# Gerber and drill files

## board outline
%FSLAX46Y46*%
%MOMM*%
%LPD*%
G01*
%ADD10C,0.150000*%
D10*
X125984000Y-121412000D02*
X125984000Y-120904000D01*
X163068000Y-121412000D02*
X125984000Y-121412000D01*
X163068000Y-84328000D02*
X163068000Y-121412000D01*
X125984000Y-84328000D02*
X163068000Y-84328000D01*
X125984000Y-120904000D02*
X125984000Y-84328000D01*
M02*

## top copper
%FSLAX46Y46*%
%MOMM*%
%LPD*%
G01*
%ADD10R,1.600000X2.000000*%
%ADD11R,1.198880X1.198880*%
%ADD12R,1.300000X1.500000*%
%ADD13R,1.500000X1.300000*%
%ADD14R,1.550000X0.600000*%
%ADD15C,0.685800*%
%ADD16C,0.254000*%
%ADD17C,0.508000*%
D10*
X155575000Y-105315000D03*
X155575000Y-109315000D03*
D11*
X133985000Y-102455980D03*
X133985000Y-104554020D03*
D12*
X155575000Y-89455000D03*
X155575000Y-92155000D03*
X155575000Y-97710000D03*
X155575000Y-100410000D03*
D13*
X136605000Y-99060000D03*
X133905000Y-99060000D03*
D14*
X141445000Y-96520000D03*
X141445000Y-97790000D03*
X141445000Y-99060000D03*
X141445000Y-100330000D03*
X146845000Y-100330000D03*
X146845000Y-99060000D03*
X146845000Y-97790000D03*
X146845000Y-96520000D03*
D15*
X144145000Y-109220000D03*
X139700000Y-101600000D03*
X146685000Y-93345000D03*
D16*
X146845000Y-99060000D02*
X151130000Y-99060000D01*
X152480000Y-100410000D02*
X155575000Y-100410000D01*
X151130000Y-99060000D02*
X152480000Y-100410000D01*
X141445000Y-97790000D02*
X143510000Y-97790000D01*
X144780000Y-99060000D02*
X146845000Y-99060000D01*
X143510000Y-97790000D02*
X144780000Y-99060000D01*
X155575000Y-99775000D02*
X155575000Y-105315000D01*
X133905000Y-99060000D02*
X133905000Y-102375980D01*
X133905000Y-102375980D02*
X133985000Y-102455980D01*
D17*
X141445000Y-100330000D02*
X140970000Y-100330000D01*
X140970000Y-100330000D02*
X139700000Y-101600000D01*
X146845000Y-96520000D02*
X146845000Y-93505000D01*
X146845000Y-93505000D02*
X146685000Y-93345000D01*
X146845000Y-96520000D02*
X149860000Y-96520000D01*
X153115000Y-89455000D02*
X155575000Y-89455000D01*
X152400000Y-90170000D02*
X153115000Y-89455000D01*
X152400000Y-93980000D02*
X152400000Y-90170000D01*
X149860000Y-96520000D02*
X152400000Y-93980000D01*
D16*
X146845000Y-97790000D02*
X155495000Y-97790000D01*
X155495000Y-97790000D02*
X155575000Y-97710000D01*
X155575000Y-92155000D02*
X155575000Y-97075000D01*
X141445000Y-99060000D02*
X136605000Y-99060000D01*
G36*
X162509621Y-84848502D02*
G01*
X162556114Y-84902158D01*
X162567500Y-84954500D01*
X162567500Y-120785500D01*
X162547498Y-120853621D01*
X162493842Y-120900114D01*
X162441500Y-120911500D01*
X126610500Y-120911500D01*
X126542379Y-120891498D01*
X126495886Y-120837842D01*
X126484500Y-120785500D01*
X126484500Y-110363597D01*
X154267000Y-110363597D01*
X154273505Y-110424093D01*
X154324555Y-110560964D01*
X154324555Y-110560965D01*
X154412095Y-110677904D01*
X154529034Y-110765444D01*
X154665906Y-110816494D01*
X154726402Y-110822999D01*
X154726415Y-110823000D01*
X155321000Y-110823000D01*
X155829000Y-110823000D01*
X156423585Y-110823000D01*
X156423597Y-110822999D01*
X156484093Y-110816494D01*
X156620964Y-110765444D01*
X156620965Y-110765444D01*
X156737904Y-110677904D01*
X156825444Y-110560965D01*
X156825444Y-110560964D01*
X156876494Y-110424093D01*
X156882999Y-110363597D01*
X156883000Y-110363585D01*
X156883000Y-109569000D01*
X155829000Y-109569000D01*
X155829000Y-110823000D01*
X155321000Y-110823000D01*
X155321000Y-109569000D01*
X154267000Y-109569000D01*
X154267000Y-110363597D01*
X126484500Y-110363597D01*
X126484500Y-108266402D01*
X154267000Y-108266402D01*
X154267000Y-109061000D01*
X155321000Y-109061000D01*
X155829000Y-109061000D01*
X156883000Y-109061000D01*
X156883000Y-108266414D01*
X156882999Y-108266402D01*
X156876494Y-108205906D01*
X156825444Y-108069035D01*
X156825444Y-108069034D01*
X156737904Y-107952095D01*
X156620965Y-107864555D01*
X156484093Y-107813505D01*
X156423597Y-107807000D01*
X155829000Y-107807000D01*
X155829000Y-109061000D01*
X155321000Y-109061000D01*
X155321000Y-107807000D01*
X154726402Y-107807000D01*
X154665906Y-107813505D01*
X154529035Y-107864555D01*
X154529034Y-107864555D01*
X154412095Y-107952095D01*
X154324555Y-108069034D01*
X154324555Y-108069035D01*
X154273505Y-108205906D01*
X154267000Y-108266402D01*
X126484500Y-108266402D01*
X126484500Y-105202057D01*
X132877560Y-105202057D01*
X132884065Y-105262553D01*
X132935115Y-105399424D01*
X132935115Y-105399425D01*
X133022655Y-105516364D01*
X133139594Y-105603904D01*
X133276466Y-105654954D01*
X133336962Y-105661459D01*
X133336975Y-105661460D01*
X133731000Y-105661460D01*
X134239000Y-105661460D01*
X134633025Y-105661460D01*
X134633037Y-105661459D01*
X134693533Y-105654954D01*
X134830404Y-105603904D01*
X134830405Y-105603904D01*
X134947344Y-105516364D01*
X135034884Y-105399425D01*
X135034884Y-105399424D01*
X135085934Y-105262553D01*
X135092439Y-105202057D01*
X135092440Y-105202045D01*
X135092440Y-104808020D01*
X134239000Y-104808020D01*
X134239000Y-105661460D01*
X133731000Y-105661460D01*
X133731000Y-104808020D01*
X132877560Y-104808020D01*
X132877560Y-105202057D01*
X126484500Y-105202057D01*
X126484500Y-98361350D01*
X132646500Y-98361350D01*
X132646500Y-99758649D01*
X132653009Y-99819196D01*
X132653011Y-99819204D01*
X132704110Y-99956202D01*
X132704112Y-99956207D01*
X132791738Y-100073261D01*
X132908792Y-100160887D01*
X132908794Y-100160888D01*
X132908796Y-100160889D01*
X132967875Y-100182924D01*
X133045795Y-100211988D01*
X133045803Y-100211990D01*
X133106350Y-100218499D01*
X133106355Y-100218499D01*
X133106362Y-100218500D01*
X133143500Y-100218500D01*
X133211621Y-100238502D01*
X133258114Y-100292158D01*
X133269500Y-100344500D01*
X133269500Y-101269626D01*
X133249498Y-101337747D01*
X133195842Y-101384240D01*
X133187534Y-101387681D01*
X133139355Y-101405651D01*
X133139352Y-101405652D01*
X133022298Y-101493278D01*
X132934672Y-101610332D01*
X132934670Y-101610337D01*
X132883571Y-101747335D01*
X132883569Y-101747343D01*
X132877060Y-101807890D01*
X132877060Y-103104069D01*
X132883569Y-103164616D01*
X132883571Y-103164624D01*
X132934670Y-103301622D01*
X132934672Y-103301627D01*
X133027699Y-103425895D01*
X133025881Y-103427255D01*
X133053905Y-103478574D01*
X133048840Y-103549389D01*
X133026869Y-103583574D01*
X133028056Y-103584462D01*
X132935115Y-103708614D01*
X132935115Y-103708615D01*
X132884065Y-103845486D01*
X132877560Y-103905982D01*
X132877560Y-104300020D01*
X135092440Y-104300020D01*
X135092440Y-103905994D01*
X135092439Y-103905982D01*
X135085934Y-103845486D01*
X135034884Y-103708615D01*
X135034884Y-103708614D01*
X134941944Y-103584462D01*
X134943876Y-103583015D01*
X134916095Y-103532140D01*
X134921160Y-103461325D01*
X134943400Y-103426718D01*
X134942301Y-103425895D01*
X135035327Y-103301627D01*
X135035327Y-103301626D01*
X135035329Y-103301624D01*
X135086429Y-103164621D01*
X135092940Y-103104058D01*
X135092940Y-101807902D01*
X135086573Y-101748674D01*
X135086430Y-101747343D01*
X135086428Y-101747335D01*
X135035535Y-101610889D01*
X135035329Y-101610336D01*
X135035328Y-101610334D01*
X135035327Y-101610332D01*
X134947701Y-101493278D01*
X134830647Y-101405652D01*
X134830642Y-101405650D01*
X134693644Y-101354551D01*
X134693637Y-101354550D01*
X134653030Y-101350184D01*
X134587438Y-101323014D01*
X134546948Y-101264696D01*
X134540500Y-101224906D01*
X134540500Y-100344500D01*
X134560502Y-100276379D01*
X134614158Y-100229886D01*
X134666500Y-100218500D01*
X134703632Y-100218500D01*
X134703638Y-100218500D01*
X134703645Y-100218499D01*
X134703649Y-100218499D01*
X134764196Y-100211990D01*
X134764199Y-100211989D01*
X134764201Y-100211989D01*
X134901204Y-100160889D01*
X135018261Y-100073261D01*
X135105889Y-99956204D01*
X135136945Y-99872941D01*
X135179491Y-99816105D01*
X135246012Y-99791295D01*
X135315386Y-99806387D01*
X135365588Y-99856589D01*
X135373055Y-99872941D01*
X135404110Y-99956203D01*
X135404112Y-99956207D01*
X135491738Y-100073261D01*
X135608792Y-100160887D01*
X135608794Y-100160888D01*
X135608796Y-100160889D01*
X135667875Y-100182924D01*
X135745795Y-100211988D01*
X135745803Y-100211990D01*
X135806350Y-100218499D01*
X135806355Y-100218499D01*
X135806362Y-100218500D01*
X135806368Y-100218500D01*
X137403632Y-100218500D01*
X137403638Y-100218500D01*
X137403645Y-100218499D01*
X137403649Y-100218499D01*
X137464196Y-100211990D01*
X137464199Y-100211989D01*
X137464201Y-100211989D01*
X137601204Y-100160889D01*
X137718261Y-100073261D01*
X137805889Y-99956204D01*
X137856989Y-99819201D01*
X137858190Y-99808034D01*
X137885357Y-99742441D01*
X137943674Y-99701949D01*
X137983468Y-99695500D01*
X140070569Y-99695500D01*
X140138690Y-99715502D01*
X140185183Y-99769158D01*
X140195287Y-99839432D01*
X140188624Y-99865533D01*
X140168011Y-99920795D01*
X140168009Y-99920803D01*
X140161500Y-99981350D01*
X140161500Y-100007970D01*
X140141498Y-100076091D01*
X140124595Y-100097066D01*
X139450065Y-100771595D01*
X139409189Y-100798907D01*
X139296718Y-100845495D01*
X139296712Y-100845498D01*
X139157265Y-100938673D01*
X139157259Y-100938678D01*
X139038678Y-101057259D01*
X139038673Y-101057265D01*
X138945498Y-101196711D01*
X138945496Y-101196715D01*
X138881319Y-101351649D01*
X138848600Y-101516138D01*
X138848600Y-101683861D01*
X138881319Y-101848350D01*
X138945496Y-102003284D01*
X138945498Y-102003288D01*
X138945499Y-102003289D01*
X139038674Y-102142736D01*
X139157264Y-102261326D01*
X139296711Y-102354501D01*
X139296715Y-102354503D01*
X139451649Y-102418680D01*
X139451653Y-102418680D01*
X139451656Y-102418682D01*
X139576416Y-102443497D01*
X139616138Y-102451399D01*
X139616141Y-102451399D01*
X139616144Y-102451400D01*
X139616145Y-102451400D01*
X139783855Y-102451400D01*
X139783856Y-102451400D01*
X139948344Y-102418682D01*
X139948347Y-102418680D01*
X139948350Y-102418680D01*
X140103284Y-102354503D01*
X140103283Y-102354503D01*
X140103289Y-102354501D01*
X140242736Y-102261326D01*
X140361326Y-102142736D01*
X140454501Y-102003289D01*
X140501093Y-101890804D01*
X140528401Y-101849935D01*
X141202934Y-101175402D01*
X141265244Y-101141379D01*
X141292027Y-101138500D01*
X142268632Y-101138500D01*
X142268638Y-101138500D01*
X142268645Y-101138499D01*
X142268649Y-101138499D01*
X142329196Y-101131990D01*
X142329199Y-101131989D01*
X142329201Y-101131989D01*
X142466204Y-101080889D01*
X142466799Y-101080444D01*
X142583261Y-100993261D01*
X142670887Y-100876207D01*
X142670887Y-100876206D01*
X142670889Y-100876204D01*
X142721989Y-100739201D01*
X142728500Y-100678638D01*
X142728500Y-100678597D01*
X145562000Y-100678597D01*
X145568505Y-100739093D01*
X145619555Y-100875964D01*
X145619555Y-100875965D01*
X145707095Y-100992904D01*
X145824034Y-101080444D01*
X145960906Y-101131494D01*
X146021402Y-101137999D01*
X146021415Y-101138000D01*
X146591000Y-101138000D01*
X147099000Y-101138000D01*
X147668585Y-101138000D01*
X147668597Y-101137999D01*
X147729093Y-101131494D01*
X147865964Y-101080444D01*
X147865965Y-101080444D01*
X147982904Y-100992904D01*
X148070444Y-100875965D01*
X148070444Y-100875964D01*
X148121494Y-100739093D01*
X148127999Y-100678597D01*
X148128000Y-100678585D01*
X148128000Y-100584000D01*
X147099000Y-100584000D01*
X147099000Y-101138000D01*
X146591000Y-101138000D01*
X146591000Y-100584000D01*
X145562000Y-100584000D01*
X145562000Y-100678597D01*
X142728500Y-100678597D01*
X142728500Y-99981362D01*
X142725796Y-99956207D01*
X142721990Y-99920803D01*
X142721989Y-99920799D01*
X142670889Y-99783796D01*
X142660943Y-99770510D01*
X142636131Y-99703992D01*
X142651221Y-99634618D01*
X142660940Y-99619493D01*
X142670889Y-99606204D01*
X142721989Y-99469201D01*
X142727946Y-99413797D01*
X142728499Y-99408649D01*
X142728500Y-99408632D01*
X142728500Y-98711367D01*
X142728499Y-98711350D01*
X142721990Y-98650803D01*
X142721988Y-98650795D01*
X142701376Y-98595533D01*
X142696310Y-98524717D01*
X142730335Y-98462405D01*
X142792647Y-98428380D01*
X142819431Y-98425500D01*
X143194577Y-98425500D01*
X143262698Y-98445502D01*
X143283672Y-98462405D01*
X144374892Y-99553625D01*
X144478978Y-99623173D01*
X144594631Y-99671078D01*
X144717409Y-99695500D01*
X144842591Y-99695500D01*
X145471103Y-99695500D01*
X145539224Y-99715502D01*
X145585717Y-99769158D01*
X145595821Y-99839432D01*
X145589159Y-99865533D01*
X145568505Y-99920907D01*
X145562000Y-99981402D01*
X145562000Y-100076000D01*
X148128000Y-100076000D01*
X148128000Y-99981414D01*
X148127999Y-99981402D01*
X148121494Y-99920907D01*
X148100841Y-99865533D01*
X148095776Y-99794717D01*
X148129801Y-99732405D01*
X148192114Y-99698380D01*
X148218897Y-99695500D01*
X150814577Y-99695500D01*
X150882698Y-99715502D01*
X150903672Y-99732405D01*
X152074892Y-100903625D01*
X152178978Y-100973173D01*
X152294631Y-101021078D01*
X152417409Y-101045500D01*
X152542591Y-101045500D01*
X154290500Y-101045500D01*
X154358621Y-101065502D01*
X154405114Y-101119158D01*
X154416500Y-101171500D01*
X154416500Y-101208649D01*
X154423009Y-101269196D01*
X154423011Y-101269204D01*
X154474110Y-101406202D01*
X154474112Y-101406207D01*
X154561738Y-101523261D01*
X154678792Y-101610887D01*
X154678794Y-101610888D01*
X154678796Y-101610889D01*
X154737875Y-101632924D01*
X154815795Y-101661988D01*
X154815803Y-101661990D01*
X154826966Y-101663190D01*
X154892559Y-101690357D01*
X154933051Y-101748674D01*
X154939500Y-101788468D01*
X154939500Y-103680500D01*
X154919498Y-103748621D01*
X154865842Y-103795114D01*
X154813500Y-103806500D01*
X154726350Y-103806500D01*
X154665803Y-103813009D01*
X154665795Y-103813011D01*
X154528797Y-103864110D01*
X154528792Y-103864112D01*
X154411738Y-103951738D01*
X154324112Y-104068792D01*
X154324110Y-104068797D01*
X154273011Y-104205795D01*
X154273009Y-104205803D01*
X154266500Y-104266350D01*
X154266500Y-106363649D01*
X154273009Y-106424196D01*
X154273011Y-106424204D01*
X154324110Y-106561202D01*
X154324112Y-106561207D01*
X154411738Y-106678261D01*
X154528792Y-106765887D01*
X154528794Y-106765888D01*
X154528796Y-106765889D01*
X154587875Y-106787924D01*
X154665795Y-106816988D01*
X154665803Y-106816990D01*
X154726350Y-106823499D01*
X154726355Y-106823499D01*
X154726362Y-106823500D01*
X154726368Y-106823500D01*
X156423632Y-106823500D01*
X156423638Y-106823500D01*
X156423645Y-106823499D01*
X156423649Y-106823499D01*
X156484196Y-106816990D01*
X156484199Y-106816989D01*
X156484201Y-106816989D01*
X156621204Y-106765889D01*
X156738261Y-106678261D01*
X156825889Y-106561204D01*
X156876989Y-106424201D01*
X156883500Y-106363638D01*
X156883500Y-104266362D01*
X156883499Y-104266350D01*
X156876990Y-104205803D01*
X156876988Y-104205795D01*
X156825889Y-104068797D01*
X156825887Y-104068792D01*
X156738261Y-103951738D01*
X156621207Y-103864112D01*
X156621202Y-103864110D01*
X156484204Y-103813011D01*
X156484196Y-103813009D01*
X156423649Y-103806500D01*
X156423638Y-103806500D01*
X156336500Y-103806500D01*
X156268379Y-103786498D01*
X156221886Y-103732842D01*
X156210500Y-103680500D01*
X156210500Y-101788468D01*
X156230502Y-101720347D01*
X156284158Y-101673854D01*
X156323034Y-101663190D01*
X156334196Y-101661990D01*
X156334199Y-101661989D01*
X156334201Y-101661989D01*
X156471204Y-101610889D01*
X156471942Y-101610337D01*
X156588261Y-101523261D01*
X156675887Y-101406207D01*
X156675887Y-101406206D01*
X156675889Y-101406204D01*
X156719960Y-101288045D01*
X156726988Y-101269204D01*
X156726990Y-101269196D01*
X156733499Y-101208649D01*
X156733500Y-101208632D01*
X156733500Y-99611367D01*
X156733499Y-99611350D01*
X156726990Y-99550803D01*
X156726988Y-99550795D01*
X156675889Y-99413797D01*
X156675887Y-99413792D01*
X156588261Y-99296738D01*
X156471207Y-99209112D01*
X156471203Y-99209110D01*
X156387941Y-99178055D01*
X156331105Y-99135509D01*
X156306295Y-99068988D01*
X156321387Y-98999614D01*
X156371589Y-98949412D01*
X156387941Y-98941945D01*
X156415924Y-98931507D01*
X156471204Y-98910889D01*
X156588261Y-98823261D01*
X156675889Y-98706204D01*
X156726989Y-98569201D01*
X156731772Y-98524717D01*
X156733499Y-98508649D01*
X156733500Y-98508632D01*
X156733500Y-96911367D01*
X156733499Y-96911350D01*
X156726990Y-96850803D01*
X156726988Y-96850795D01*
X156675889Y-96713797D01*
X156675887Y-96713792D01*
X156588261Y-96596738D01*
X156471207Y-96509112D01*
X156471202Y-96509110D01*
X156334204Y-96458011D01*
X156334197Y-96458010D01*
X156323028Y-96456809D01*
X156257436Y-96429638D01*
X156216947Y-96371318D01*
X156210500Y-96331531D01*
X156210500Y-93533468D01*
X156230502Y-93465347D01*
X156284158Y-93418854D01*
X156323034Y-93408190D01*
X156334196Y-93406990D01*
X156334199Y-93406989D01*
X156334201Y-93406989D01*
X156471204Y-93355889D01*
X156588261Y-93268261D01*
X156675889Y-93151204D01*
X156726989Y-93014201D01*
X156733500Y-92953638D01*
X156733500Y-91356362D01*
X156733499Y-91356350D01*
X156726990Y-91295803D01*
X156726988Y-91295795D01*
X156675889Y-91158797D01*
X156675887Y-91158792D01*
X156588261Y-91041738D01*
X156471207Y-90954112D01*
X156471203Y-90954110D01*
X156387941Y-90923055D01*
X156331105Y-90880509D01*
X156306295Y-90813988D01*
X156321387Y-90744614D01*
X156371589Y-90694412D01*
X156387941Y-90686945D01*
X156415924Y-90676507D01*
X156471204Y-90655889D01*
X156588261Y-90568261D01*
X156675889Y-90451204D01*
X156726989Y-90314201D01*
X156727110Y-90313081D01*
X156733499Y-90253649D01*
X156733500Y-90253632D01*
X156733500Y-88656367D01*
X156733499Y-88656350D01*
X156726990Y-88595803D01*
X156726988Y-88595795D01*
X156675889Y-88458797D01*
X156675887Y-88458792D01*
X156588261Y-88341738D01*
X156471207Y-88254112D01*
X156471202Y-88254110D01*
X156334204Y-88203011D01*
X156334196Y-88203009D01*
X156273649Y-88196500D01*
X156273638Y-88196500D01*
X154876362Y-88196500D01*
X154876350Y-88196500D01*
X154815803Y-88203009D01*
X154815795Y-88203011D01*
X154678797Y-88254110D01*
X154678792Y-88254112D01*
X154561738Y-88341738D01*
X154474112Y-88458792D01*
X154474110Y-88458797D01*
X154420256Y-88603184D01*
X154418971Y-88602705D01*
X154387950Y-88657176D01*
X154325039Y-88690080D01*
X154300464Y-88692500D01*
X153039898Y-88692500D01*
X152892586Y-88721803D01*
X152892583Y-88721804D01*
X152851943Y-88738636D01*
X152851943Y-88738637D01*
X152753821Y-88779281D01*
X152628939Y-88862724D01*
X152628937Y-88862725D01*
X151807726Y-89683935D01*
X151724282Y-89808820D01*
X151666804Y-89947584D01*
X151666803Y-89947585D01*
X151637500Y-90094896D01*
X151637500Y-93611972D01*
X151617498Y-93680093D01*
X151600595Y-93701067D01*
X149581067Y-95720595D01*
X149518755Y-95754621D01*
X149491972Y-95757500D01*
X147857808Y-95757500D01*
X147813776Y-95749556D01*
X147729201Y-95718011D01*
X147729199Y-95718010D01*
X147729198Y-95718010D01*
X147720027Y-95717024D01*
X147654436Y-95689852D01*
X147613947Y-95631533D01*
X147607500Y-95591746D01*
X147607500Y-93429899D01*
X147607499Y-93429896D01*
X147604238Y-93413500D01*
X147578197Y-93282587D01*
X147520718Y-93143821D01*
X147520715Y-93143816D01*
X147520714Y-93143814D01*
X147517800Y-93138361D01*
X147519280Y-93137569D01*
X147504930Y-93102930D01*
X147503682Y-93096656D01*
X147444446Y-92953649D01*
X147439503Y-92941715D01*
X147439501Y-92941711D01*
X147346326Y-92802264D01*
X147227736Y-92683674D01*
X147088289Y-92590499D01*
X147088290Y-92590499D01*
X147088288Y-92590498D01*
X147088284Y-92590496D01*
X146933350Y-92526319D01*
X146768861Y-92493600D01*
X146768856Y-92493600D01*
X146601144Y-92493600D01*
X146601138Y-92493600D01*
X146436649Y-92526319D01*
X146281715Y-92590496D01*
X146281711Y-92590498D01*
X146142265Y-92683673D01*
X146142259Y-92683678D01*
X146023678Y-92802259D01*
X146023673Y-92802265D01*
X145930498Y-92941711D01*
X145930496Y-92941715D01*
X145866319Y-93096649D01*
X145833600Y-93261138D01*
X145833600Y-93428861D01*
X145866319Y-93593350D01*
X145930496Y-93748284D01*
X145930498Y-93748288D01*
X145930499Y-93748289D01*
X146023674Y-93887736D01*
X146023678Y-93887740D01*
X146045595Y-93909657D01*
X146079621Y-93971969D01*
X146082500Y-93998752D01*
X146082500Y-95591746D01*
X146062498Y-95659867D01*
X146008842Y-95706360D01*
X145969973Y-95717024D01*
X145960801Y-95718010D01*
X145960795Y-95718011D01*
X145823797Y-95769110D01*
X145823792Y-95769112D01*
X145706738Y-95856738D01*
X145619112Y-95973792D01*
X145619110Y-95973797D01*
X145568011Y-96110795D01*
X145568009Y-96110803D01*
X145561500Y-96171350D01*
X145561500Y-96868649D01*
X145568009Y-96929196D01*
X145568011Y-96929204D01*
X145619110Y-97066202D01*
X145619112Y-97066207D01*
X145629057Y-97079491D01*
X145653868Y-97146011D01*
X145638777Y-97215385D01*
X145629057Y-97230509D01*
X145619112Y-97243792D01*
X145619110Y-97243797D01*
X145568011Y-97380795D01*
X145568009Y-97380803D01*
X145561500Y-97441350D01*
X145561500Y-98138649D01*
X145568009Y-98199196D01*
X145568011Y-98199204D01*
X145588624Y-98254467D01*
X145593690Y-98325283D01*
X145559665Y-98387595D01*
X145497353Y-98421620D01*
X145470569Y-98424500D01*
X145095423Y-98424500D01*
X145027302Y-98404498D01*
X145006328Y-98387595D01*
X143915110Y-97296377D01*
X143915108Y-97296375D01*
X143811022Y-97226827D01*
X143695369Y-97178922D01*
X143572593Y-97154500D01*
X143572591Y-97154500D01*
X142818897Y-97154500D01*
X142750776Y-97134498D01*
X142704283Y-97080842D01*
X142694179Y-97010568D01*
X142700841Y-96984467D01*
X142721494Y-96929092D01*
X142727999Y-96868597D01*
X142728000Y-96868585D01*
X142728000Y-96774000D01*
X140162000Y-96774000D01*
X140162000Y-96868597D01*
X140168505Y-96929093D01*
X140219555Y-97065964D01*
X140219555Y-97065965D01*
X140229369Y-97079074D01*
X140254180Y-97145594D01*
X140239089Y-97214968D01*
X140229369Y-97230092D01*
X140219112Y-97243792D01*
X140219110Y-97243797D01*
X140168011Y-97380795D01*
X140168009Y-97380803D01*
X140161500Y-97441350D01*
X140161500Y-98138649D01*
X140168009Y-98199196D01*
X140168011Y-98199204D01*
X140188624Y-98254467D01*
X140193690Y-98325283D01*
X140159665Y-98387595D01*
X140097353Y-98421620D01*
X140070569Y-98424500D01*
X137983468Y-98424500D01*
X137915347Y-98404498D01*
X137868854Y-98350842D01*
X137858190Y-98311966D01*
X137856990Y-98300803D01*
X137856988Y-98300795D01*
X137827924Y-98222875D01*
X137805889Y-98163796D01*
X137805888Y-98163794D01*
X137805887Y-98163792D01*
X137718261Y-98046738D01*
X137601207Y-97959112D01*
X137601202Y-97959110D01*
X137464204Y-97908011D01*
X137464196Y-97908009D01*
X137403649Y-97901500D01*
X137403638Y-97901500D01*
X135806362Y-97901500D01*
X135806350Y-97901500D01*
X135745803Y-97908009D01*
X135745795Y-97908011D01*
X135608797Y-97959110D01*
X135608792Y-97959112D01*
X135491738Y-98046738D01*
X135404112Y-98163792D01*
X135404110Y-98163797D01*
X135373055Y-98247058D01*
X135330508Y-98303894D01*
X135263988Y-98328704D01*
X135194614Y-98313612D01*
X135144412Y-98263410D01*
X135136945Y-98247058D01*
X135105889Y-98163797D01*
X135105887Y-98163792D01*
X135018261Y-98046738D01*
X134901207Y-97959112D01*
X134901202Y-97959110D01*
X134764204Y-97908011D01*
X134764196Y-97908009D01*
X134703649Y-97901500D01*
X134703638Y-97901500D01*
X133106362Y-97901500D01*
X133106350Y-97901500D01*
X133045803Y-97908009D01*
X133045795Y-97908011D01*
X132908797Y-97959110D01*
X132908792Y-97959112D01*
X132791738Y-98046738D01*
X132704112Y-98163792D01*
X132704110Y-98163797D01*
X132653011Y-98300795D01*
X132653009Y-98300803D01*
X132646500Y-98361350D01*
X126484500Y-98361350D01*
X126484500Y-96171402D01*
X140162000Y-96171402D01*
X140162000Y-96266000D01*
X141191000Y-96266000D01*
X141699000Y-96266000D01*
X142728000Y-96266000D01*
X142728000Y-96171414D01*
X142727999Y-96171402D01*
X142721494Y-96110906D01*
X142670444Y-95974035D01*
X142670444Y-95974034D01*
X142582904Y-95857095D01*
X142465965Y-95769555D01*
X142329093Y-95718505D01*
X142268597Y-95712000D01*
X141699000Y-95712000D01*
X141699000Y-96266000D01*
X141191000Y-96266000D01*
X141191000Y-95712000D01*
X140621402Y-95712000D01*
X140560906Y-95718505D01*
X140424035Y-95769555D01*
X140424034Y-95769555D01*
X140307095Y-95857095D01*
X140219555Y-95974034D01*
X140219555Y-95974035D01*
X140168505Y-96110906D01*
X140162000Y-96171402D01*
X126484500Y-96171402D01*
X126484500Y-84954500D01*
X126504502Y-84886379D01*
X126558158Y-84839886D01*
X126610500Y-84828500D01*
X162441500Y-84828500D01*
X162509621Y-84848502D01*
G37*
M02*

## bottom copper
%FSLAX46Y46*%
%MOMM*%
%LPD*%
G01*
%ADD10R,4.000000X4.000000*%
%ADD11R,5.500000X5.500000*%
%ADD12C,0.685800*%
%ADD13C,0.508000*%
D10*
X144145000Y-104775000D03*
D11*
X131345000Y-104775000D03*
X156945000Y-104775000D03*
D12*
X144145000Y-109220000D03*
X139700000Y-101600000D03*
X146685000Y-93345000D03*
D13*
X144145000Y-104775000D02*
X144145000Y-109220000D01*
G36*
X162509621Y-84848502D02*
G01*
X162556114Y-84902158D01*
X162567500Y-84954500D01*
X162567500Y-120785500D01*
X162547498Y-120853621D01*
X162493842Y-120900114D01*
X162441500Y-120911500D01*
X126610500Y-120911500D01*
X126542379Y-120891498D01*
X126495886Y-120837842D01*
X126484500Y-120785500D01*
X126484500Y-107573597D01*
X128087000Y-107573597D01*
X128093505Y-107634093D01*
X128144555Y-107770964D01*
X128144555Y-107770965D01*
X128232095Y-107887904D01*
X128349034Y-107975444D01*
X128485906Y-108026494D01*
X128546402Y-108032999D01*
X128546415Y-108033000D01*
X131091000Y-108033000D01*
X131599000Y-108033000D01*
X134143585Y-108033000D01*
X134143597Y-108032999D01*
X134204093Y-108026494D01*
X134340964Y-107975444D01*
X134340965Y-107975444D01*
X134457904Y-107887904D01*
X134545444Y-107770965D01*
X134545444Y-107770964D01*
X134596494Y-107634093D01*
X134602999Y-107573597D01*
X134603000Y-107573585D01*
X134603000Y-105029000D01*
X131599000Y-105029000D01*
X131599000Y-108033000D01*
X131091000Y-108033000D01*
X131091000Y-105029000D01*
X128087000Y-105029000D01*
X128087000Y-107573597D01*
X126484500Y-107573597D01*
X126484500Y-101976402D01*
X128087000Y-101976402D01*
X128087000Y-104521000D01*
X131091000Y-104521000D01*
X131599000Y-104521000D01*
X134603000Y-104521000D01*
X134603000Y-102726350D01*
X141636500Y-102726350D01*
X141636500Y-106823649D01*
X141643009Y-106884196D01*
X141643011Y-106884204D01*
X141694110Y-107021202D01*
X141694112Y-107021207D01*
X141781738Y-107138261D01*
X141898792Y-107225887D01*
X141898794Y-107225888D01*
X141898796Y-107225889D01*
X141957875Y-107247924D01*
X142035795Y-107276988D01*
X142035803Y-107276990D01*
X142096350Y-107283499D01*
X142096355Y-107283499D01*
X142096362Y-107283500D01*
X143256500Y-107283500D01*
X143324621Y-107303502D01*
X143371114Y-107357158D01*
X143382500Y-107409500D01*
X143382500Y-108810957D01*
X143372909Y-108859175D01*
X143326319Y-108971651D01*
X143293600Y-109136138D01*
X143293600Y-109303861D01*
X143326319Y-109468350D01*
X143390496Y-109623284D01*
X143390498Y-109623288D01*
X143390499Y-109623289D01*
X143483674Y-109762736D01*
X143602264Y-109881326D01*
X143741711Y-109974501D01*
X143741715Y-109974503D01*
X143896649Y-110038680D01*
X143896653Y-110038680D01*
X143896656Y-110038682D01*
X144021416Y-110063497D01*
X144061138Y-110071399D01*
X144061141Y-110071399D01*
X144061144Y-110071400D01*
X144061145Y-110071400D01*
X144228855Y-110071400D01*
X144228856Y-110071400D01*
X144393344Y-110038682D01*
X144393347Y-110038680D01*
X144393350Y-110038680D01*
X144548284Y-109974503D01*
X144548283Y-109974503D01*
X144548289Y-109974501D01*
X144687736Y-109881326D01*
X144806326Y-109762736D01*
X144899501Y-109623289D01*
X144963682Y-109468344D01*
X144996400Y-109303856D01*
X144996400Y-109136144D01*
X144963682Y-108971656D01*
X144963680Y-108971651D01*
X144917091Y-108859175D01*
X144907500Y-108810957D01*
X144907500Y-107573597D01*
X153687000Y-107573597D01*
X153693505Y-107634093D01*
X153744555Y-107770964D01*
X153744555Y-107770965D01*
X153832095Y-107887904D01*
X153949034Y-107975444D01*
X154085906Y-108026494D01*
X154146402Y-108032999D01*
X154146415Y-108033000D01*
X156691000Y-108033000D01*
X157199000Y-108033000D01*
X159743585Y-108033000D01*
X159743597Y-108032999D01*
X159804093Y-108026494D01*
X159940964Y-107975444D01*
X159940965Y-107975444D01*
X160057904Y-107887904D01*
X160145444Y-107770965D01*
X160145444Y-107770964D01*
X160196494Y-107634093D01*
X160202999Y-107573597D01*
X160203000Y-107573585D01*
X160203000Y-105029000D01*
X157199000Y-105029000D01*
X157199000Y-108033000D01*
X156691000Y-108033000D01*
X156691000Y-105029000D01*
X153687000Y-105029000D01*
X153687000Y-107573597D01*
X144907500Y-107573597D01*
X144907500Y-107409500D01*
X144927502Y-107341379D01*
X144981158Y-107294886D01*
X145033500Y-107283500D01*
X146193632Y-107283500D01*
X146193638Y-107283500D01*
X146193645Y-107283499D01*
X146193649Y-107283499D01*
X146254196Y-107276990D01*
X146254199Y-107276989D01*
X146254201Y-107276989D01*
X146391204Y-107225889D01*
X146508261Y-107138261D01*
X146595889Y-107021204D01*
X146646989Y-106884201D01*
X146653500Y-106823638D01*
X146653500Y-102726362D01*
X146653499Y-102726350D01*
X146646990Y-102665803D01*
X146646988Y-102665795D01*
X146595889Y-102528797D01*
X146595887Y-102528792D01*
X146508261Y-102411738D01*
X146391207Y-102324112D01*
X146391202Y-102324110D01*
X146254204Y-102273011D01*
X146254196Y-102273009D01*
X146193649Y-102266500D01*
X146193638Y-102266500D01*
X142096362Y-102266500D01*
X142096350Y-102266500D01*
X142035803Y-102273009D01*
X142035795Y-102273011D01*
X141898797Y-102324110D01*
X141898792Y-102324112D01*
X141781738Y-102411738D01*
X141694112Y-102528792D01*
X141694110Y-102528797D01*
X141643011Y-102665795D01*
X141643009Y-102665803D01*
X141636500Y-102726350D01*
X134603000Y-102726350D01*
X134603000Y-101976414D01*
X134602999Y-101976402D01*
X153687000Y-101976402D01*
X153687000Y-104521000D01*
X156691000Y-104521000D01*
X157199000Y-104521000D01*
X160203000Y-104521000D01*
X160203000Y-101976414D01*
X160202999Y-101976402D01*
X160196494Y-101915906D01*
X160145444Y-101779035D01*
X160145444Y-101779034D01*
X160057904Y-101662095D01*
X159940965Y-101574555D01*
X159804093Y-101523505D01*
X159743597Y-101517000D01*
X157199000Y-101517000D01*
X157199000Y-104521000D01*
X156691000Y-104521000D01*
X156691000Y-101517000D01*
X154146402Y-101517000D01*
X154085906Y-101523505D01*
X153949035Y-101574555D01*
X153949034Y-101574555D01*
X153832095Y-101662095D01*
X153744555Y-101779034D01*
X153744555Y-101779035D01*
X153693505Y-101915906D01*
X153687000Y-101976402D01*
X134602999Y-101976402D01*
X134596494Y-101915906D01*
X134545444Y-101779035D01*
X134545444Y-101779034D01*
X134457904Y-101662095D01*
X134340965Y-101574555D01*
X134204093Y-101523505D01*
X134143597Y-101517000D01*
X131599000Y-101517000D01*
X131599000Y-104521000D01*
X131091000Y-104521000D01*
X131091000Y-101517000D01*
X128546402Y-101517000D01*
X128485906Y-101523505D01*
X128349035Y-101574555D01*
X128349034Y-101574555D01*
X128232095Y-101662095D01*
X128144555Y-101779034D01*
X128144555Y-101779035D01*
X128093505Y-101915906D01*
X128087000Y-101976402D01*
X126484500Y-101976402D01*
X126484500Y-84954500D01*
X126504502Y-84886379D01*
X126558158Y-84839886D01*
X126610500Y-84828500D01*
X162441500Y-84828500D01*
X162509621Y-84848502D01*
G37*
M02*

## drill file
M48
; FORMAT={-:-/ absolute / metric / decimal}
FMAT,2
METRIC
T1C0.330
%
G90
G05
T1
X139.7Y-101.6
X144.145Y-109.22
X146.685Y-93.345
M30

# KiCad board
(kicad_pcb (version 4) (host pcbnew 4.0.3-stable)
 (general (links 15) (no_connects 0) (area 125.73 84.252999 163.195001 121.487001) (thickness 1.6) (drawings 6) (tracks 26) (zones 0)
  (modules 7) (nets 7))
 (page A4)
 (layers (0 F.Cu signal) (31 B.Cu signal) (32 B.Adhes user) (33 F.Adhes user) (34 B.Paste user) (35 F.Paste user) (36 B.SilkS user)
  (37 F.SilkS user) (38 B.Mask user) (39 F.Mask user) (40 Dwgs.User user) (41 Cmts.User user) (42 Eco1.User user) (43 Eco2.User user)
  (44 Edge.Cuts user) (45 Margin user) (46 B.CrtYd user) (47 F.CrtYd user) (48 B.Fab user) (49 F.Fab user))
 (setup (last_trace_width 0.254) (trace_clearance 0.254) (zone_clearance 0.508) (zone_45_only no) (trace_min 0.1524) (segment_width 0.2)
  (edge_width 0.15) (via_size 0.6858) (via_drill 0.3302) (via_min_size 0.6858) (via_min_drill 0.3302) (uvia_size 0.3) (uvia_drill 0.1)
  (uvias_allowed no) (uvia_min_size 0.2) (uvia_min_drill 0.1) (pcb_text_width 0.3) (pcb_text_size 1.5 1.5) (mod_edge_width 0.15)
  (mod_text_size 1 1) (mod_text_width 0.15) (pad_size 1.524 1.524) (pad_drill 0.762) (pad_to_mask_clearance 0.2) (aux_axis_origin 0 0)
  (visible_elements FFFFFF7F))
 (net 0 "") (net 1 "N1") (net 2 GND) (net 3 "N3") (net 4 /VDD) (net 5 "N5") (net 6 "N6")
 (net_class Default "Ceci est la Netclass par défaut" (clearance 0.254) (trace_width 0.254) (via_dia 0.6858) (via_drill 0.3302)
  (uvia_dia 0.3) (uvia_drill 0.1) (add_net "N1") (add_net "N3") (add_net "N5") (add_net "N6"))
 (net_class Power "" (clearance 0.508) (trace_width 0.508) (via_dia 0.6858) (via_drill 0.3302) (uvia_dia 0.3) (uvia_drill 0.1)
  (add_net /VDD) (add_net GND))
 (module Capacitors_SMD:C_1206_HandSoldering (layer F.Cu) (at 155.575 107.315 270)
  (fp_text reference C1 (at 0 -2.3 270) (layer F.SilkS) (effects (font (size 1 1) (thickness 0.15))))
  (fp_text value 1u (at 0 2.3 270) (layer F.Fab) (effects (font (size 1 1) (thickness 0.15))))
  (pad 1 smd rect (at -2 0 270) (size 2 1.6) (layers F.Cu F.Paste F.Mask) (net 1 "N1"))
  (pad 2 smd rect (at 2 0 270) (size 2 1.6) (layers F.Cu F.Paste F.Mask) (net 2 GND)))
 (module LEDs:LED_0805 (layer F.Cu) (at 133.985 103.505 90)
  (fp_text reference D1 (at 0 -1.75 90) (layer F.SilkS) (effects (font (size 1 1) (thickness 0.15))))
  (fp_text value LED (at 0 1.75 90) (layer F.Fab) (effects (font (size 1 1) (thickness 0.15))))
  (pad 2 smd rect (at 1.04902 0 270) (size 1.19888 1.19888) (layers F.Cu F.Paste F.Mask) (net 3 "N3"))
  (pad 1 smd rect (at -1.04902 0 270) (size 1.19888 1.19888) (layers F.Cu F.Paste F.Mask) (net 2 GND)))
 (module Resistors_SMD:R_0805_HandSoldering (layer F.Cu) (at 155.575 90.805 270)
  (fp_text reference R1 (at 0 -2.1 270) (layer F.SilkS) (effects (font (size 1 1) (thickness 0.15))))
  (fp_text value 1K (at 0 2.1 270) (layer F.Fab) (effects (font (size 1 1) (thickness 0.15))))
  (pad 1 smd rect (at -1.35 0 270) (size 1.5 1.3) (layers F.Cu F.Paste F.Mask) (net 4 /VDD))
  (pad 2 smd rect (at 1.35 0 270) (size 1.5 1.3) (layers F.Cu F.Paste F.Mask) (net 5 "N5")))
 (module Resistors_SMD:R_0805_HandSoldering (layer F.Cu) (at 155.575 99.06 270)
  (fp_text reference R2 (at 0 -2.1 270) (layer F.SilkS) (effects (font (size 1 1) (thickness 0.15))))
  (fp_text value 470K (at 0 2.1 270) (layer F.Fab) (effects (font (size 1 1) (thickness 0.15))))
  (pad 1 smd rect (at -1.35 0 270) (size 1.5 1.3) (layers F.Cu F.Paste F.Mask) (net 5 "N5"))
  (pad 2 smd rect (at 1.35 0 270) (size 1.5 1.3) (layers F.Cu F.Paste F.Mask) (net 1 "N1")))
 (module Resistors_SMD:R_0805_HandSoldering (layer F.Cu) (at 135.255 99.06 180)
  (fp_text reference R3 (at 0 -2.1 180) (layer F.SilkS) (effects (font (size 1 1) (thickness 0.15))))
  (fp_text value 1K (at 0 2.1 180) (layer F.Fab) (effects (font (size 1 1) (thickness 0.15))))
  (pad 1 smd rect (at -1.35 0 180) (size 1.5 1.3) (layers F.Cu F.Paste F.Mask) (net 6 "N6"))
  (pad 2 smd rect (at 1.35 0 180) (size 1.5 1.3) (layers F.Cu F.Paste F.Mask) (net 3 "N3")))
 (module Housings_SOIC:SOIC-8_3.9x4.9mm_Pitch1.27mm (layer F.Cu) (at 144.145 98.425)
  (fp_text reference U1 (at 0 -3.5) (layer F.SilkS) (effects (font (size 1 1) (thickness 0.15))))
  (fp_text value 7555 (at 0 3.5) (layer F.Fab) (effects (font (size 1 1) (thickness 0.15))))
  (pad 1 smd rect (at -2.7 -1.905) (size 1.55 0.6) (layers F.Cu F.Paste F.Mask) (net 2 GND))
  (pad 2 smd rect (at -2.7 -0.635) (size 1.55 0.6) (layers F.Cu F.Paste F.Mask) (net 1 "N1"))
  (pad 3 smd rect (at -2.7 0.635) (size 1.55 0.6) (layers F.Cu F.Paste F.Mask) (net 6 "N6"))
  (pad 4 smd rect (at -2.7 1.905) (size 1.55 0.6) (layers F.Cu F.Paste F.Mask) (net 4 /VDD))
  (pad 5 smd rect (at 2.7 1.905) (size 1.55 0.6) (layers F.Cu F.Paste F.Mask) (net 2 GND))
  (pad 6 smd rect (at 2.7 0.635) (size 1.55 0.6) (layers F.Cu F.Paste F.Mask) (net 1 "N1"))
  (pad 7 smd rect (at 2.7 -0.635) (size 1.55 0.6) (layers F.Cu F.Paste F.Mask) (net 5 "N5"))
  (pad 8 smd rect (at 2.7 -1.905) (size 1.55 0.6) (layers F.Cu F.Paste F.Mask) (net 4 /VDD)))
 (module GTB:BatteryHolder (layer B.Cu) (at 144.145 104.775)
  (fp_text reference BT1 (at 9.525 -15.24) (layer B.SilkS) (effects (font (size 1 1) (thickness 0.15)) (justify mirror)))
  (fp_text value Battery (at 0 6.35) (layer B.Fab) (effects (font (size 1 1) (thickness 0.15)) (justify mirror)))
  (pad 2 smd rect (at 0 0) (size 4 4) (layers B.Cu B.Paste B.Mask) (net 2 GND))
  (pad 1 smd rect (at -12.8 0) (size 5.5 5.5) (layers B.Cu B.Paste B.Mask) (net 4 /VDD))
  (pad 1 smd rect (at 12.8 0) (size 5.5 5.5) (layers B.Cu B.Paste B.Mask) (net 4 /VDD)))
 (gr_line (start 125.984 121.412) (end 125.984 120.904) (angle 90) (layer Edge.Cuts) (width 0.15))
 (gr_line (start 163.068 121.412) (end 125.984 121.412) (angle 90) (layer Edge.Cuts) (width 0.15))
 (gr_line (start 163.068 84.328) (end 163.068 121.412) (angle 90) (layer Edge.Cuts) (width 0.15))
 (gr_line (start 125.984 84.328) (end 163.068 84.328) (angle 90) (layer Edge.Cuts) (width 0.15))
 (gr_line (start 125.984 120.904) (end 125.984 84.328) (angle 90) (layer Edge.Cuts) (width 0.15))
 (segment (start 146.845 99.06) (end 151.13 99.06) (width 0.254) (layer F.Cu) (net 1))
 (segment (start 152.48 100.41) (end 155.575 100.41) (width 0.254) (layer F.Cu) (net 1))
 (segment (start 151.13 99.06) (end 152.48 100.41) (width 0.254) (layer F.Cu) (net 1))
 (segment (start 141.445 97.79) (end 143.51 97.79) (width 0.254) (layer F.Cu) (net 1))
 (segment (start 144.78 99.06) (end 146.845 99.06) (width 0.254) (layer F.Cu) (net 1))
 (segment (start 143.51 97.79) (end 144.78 99.06) (width 0.254) (layer F.Cu) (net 1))
 (segment (start 155.575 99.775) (end 155.575 105.315) (width 0.254) (layer F.Cu) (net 1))
 (segment (start 144.145 104.775) (end 144.145 109.22) (width 0.508) (layer B.Cu) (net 2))
 (via (at 144.145 109.22) (size 0.6858) (drill 0.3302) (layers F.Cu B.Cu) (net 2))
 (segment (start 133.905 99.06) (end 133.905 102.37598) (width 0.254) (layer F.Cu) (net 3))
 (segment (start 133.905 102.37598) (end 133.985 102.45598) (width 0.254) (layer F.Cu) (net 3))
 (segment (start 141.445 100.33) (end 140.97 100.33) (width 0.508) (layer F.Cu) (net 4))
 (segment (start 140.97 100.33) (end 139.7 101.6) (width 0.508) (layer F.Cu) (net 4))
 (via (at 139.7 101.6) (size 0.6858) (drill 0.3302) (layers F.Cu B.Cu) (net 4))
 (segment (start 146.845 96.52) (end 146.845 93.505) (width 0.508) (layer F.Cu) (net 4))
 (via (at 146.685 93.345) (size 0.6858) (drill 0.3302) (layers F.Cu B.Cu) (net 4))
 (segment (start 146.845 93.505) (end 146.685 93.345) (width 0.508) (layer F.Cu) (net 4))
 (segment (start 146.845 96.52) (end 149.86 96.52) (width 0.508) (layer F.Cu) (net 4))
 (segment (start 153.115 89.455) (end 155.575 89.455) (width 0.508) (layer F.Cu) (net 4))
 (segment (start 152.4 90.17) (end 153.115 89.455) (width 0.508) (layer F.Cu) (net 4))
 (segment (start 152.4 93.98) (end 152.4 90.17) (width 0.508) (layer F.Cu) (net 4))
 (segment (start 149.86 96.52) (end 152.4 93.98) (width 0.508) (layer F.Cu) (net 4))
 (segment (start 146.845 97.79) (end 155.495 97.79) (width 0.254) (layer F.Cu) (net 5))
 (segment (start 155.495 97.79) (end 155.575 97.71) (width 0.254) (layer F.Cu) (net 5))
 (segment (start 155.575 92.155) (end 155.575 97.075) (width 0.254) (layer F.Cu) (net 5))
 (segment (start 141.445 99.06) (end 136.605 99.06) (width 0.254) (layer F.Cu) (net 6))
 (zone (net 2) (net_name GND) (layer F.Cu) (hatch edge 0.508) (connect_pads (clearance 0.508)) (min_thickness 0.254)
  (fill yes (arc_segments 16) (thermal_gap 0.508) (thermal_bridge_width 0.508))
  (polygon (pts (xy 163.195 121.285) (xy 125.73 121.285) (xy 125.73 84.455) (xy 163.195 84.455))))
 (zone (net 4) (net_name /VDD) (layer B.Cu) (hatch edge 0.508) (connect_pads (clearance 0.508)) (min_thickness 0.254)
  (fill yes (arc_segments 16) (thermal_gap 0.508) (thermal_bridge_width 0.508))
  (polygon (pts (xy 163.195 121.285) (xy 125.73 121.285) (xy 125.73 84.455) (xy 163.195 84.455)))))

